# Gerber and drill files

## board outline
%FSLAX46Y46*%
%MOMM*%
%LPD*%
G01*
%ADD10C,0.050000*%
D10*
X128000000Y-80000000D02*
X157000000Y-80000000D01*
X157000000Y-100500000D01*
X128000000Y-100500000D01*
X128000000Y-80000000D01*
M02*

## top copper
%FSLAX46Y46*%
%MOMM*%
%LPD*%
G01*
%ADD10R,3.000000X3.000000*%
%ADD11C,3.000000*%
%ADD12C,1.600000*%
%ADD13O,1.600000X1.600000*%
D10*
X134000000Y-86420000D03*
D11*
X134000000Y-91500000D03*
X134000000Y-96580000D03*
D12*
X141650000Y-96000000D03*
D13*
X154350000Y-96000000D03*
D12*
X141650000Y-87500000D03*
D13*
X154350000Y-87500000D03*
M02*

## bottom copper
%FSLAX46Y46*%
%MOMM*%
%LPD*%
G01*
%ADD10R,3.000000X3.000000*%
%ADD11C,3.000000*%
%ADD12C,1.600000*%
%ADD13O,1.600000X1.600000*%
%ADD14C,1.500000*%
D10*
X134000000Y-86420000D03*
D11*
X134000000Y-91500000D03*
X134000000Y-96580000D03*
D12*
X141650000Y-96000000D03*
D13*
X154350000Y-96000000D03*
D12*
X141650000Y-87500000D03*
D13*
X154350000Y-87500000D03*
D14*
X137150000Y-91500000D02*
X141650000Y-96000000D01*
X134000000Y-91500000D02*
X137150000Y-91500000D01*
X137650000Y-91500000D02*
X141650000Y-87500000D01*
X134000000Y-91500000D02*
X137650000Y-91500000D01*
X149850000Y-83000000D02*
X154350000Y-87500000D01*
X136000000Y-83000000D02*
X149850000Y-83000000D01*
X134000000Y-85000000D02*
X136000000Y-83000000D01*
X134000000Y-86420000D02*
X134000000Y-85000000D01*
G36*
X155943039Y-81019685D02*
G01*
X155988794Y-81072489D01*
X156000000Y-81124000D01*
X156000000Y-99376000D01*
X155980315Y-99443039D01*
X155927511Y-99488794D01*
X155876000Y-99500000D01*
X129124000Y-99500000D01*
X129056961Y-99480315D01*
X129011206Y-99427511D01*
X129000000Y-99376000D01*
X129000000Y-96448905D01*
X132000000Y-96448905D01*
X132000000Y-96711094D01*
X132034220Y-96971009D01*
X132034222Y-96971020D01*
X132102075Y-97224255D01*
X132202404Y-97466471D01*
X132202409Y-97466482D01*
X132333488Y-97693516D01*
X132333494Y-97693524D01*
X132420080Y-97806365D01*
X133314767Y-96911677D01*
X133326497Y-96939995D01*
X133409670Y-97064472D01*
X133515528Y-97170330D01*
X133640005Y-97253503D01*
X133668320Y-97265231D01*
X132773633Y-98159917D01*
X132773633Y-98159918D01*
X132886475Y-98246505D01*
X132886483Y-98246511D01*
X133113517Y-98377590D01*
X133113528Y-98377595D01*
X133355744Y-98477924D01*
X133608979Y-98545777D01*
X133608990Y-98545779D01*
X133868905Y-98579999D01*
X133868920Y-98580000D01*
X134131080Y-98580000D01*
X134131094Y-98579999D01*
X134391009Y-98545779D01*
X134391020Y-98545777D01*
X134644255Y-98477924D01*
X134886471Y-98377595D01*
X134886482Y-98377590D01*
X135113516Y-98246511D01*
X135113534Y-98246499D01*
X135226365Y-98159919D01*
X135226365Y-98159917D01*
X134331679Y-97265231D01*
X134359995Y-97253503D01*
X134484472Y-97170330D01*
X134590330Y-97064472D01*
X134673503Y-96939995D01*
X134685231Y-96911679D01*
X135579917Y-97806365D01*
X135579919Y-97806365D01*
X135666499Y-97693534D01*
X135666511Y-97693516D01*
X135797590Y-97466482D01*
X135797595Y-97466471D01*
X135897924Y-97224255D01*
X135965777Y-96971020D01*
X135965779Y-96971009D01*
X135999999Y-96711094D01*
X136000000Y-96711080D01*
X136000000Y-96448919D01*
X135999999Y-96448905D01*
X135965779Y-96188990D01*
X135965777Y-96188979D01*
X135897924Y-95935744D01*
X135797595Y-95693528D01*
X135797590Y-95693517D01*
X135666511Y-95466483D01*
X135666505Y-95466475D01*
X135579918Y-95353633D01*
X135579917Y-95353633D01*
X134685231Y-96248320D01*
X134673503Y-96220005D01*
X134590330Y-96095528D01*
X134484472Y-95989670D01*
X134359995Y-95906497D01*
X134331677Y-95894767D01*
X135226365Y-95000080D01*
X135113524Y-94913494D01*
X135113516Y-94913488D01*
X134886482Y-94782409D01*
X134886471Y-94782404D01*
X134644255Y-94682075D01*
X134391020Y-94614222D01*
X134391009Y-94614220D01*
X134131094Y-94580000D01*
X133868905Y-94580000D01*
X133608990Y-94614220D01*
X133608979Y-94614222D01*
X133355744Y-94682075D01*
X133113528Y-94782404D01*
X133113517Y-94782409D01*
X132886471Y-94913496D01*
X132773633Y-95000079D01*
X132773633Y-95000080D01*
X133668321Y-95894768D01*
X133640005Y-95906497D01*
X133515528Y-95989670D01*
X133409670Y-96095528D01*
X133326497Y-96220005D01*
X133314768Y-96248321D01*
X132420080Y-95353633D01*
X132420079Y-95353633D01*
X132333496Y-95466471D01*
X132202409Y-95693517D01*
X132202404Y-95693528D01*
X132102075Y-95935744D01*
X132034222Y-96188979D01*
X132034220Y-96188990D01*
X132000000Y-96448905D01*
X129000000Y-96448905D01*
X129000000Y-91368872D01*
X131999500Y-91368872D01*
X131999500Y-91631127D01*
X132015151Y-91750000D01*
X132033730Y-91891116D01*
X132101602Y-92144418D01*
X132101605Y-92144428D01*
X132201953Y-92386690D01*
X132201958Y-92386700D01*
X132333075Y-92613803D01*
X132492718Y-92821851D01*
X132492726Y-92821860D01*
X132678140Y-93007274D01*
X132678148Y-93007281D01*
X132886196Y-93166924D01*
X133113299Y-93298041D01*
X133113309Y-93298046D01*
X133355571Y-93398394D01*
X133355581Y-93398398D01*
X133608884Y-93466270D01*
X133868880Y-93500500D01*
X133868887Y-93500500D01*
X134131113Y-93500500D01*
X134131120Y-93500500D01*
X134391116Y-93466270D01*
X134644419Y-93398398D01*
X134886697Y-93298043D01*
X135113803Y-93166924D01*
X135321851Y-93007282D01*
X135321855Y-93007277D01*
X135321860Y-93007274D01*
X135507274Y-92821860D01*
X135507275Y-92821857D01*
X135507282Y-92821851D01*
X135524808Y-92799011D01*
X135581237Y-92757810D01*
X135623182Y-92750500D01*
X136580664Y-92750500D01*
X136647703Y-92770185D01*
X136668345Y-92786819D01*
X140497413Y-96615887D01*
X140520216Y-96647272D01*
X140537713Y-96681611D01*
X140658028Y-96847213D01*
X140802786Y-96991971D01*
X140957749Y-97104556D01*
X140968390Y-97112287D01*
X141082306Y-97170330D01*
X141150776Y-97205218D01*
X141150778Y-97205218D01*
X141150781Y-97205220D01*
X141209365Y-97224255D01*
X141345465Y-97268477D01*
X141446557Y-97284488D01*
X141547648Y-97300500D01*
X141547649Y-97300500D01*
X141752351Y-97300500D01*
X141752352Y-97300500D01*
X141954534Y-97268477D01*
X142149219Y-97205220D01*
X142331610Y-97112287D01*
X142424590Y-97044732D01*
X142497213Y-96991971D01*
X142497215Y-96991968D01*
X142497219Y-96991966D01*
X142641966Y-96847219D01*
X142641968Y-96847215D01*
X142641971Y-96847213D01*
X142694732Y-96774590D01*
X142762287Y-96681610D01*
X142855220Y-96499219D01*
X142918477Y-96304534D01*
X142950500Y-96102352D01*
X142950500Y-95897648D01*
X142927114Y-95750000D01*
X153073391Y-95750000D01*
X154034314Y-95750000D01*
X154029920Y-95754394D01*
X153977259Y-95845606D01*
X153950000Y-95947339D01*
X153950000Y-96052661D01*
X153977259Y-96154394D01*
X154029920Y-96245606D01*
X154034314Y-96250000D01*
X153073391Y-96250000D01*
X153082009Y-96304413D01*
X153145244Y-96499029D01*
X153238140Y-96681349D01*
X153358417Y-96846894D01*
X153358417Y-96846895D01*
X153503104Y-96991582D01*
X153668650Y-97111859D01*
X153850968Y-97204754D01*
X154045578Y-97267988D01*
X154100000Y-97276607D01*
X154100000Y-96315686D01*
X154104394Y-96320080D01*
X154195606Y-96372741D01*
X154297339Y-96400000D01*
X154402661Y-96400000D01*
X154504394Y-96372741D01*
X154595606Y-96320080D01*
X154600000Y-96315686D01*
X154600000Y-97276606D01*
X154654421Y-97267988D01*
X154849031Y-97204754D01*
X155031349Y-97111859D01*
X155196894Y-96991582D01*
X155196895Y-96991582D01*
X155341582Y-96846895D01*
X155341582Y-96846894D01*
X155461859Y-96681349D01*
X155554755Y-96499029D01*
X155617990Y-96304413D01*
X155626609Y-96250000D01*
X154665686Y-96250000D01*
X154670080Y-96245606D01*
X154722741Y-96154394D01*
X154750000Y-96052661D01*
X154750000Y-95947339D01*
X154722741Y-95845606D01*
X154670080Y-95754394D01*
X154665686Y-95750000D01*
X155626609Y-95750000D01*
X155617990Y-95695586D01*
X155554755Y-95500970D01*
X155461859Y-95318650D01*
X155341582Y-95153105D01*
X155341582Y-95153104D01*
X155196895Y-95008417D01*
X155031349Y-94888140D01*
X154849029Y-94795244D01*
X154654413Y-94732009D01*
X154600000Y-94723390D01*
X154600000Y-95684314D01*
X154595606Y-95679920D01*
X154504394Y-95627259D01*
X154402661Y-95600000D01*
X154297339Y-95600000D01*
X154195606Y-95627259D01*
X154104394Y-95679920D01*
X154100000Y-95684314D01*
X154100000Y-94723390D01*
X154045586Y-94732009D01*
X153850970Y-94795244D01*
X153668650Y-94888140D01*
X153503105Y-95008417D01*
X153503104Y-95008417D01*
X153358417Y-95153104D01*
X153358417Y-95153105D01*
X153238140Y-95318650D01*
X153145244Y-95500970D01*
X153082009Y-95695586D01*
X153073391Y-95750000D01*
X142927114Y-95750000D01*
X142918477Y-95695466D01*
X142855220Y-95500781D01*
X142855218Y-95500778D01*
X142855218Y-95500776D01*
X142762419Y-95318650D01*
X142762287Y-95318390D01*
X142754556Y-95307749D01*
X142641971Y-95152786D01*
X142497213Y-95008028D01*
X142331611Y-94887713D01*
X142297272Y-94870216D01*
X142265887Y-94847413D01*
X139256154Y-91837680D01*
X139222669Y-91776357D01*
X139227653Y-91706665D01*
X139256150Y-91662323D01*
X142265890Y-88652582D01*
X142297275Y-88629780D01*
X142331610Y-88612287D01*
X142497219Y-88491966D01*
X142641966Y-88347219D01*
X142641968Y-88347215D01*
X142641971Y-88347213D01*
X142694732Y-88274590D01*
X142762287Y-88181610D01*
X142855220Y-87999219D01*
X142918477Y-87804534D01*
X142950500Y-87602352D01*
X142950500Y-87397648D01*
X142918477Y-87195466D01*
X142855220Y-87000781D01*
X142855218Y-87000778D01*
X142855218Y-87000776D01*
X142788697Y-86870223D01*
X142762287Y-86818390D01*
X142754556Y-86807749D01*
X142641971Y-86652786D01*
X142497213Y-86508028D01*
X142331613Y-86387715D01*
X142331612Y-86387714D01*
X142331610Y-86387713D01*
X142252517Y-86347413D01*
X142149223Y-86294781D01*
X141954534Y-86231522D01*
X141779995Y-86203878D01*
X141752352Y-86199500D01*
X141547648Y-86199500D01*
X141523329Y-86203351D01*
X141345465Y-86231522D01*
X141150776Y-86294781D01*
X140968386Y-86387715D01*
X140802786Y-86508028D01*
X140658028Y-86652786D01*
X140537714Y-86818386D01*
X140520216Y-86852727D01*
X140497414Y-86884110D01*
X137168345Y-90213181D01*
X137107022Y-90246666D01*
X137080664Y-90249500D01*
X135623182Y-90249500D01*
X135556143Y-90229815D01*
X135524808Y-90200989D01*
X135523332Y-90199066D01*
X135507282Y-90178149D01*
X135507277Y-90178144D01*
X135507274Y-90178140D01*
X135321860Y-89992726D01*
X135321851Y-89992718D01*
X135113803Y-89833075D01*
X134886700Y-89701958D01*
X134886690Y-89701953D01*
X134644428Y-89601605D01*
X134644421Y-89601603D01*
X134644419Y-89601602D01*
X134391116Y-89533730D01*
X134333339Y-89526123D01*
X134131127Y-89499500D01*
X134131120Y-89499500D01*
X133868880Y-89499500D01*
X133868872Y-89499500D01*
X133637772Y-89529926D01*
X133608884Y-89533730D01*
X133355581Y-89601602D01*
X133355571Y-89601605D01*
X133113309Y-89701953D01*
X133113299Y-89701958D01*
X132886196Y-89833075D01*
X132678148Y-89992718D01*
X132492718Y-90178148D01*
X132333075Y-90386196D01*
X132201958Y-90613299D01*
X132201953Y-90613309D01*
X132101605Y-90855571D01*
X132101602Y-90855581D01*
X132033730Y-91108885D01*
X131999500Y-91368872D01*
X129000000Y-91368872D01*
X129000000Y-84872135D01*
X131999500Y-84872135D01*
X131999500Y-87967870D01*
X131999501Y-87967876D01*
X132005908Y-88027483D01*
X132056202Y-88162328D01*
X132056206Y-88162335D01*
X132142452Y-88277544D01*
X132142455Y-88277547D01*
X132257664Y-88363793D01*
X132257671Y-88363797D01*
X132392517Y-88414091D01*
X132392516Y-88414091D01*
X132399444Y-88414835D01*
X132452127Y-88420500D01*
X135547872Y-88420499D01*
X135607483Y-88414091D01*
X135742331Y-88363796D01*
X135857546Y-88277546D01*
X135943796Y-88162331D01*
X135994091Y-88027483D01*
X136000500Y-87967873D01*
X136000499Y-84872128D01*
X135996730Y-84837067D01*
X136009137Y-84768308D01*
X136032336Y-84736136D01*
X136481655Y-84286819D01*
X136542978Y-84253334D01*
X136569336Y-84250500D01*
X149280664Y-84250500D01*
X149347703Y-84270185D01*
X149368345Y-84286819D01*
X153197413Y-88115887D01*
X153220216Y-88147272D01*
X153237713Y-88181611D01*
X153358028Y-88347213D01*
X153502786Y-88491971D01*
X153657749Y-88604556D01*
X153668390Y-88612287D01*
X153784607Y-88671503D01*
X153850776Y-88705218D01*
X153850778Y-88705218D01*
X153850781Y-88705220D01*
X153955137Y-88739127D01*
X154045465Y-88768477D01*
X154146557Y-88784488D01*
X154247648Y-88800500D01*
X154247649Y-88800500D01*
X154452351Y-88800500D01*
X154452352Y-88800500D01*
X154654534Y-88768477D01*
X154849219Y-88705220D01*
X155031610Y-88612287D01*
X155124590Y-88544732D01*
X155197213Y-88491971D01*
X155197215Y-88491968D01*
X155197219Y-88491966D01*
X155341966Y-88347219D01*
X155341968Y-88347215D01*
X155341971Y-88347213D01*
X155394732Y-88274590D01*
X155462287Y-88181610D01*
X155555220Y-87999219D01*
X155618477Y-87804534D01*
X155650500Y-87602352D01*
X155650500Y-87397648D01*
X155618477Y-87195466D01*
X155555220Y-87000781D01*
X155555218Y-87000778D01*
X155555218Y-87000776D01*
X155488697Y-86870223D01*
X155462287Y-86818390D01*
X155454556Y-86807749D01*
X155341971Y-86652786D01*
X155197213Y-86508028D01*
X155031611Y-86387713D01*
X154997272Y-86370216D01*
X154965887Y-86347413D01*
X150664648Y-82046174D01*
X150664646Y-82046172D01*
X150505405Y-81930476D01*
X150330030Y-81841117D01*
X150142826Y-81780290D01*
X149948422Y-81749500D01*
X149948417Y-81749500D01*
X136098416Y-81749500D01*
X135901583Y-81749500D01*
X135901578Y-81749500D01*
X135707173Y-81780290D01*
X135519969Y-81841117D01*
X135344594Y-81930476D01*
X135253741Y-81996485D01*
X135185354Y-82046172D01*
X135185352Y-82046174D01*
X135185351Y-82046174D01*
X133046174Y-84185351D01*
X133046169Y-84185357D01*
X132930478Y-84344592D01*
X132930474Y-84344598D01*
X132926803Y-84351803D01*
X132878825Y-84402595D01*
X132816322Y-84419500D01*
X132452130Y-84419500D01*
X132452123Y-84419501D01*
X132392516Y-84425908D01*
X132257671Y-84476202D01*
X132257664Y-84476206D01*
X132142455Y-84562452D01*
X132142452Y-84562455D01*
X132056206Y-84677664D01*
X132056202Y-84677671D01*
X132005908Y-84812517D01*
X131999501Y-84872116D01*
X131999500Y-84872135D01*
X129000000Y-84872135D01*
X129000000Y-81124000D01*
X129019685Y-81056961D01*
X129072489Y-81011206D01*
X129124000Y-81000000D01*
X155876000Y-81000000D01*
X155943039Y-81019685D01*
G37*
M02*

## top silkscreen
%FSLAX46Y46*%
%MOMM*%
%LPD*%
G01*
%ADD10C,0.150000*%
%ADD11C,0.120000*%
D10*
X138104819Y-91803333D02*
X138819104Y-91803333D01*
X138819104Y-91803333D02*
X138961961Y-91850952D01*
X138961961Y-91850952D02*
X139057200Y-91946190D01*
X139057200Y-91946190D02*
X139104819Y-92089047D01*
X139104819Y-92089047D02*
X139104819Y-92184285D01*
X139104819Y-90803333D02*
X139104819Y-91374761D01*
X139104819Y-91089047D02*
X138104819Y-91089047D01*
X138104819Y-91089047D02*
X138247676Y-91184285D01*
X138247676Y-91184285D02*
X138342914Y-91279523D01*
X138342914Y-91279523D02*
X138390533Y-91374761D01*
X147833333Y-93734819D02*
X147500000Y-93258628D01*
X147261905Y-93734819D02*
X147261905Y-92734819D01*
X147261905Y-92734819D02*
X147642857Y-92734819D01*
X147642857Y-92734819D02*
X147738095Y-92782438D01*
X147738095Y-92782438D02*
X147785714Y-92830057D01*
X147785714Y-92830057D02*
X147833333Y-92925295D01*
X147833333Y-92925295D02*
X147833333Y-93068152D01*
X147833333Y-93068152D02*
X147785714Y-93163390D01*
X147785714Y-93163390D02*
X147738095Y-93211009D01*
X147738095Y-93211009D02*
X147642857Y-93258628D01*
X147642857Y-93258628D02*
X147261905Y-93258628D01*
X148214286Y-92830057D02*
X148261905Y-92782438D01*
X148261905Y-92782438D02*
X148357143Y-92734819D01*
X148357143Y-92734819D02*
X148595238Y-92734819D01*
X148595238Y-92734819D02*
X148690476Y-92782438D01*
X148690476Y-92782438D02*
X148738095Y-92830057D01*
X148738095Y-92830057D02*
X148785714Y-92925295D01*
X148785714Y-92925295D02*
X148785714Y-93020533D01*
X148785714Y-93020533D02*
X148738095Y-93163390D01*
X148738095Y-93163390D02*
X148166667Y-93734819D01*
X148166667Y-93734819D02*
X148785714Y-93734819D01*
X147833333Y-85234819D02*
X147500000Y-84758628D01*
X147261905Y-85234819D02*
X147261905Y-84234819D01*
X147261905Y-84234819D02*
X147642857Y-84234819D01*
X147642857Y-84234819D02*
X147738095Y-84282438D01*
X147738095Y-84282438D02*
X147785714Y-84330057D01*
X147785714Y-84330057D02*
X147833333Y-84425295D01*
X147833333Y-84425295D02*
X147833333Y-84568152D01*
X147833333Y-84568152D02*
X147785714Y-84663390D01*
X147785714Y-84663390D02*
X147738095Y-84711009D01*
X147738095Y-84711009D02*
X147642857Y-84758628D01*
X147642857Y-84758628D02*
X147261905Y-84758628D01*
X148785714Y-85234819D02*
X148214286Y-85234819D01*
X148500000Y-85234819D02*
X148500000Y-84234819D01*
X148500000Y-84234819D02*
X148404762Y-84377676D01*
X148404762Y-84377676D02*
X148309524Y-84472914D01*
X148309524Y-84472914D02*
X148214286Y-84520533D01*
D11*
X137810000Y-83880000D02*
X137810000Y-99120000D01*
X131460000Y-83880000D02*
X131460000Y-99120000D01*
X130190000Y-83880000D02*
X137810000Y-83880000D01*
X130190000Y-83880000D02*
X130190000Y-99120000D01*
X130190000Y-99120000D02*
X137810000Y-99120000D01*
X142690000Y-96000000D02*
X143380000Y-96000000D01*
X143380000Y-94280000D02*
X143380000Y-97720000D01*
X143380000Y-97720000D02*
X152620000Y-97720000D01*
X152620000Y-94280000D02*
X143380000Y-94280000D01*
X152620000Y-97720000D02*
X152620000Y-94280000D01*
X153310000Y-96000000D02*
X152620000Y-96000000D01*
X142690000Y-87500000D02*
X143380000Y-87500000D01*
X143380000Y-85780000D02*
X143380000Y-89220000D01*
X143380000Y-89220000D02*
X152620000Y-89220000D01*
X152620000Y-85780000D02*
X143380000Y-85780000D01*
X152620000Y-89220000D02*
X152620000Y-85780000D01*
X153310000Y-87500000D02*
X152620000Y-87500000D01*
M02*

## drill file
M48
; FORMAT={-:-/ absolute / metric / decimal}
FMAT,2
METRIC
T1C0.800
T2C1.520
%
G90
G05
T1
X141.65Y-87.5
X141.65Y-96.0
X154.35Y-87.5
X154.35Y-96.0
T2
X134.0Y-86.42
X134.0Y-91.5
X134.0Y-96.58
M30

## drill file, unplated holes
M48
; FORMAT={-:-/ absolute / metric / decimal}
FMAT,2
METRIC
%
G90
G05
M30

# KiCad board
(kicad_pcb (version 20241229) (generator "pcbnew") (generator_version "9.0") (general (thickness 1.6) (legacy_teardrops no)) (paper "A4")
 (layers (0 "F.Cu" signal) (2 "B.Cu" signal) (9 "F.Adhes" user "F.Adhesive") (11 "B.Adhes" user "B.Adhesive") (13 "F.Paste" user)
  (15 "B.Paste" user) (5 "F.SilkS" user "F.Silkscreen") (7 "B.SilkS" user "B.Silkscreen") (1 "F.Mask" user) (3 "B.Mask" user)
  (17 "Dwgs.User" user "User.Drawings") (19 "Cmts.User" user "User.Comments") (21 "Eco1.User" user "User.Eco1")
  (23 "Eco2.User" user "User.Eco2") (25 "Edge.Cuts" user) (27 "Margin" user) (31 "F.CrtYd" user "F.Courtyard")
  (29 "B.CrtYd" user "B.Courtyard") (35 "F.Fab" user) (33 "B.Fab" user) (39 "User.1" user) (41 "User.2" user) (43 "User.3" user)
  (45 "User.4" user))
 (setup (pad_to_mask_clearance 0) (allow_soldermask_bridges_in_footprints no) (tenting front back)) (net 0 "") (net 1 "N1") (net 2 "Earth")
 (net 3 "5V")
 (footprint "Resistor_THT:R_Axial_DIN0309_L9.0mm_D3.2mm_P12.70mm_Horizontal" (layer "F.Cu") (at 141.65 96)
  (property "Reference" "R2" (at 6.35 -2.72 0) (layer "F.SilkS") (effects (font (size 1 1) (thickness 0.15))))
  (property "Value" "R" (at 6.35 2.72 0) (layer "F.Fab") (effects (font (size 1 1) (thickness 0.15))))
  (fp_line (start 1.04 0) (end 1.73 0) (stroke (width 0.12) (type solid)) (layer "F.SilkS"))
  (fp_line (start 1.73 -1.72) (end 1.73 1.72) (stroke (width 0.12) (type solid)) (layer "F.SilkS"))
  (fp_line (start 1.73 1.72) (end 10.97 1.72) (stroke (width 0.12) (type solid)) (layer "F.SilkS"))
  (fp_line (start 10.97 -1.72) (end 1.73 -1.72) (stroke (width 0.12) (type solid)) (layer "F.SilkS"))
  (fp_line (start 10.97 1.72) (end 10.97 -1.72) (stroke (width 0.12) (type solid)) (layer "F.SilkS"))
  (fp_line (start 11.66 0) (end 10.97 0) (stroke (width 0.12) (type solid)) (layer "F.SilkS"))
  (pad "1" thru_hole circle (at 0 0) (size 1.6 1.6) (drill 0.8) (layers "*.Cu" "*.Mask") (remove_unused_layers no) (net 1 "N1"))
  (pad "2" thru_hole oval (at 12.7 0) (size 1.6 1.6) (drill 0.8) (layers "*.Cu" "*.Mask") (remove_unused_layers no) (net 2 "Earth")))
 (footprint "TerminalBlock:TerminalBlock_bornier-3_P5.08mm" (layer "F.Cu") (at 134 86.42 -90)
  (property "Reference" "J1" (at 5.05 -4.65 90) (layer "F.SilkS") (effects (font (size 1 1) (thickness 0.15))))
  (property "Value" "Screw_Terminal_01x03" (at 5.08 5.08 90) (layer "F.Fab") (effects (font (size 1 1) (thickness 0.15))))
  (fp_line (start -2.54 3.81) (end 12.7 3.81) (stroke (width 0.12) (type solid)) (layer "F.SilkS"))
  (fp_line (start -2.54 3.81) (end -2.54 -3.81) (stroke (width 0.12) (type solid)) (layer "F.SilkS"))
  (fp_line (start 12.7 3.81) (end 12.7 -3.81) (stroke (width 0.12) (type solid)) (layer "F.SilkS"))
  (fp_line (start -2.54 2.54) (end 12.7 2.54) (stroke (width 0.12) (type solid)) (layer "F.SilkS"))
  (fp_line (start -2.54 -3.81) (end 12.7 -3.81) (stroke (width 0.12) (type solid)) (layer "F.SilkS"))
  (pad "1" thru_hole rect (at 0 0 270) (size 3 3) (drill 1.52) (layers "*.Cu" "*.Mask") (remove_unused_layers no) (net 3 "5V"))
  (pad "2" thru_hole circle (at 5.08 0 270) (size 3 3) (drill 1.52) (layers "*.Cu" "*.Mask") (remove_unused_layers no) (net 1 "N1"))
  (pad "3" thru_hole circle (at 10.16 0 270) (size 3 3) (drill 1.52) (layers "*.Cu" "*.Mask") (remove_unused_layers no) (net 2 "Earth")))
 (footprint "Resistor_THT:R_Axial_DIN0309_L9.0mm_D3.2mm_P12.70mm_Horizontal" (layer "F.Cu") (at 141.65 87.5)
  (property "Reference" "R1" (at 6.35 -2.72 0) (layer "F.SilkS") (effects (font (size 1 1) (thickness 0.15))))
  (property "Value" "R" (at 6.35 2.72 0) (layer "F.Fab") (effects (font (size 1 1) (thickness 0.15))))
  (fp_line (start 1.04 0) (end 1.73 0) (stroke (width 0.12) (type solid)) (layer "F.SilkS"))
  (fp_line (start 1.73 -1.72) (end 1.73 1.72) (stroke (width 0.12) (type solid)) (layer "F.SilkS"))
  (fp_line (start 1.73 1.72) (end 10.97 1.72) (stroke (width 0.12) (type solid)) (layer "F.SilkS"))
  (fp_line (start 10.97 -1.72) (end 1.73 -1.72) (stroke (width 0.12) (type solid)) (layer "F.SilkS"))
  (fp_line (start 10.97 1.72) (end 10.97 -1.72) (stroke (width 0.12) (type solid)) (layer "F.SilkS"))
  (fp_line (start 11.66 0) (end 10.97 0) (stroke (width 0.12) (type solid)) (layer "F.SilkS"))
  (pad "1" thru_hole circle (at 0 0) (size 1.6 1.6) (drill 0.8) (layers "*.Cu" "*.Mask") (remove_unused_layers no) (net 1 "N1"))
  (pad "2" thru_hole oval (at 12.7 0) (size 1.6 1.6) (drill 0.8) (layers "*.Cu" "*.Mask") (remove_unused_layers no) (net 3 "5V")))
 (gr_rect (start 128 80) (end 157 100.5) (stroke (width 0.05) (type default)) (fill no) (layer "Edge.Cuts"))
 (segment (start 134 85) (end 136 83) (width 1.5) (layer "B.Cu") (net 3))
 (segment (start 134 86.42) (end 134 85) (width 1.5) (layer "B.Cu") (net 3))
 (segment (start 136 83) (end 149.85 83) (width 1.5) (layer "B.Cu") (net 3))
 (segment (start 149.85 83) (end 154.35 87.5) (width 1.5) (layer "B.Cu") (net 3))
 (segment (start 137.15 91.5) (end 141.65 96) (width 1.5) (layer "B.Cu") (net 1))
 (segment (start 137.65 91.5) (end 141.65 87.5) (width 1.5) (layer "B.Cu") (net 1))
 (segment (start 134 91.5) (end 137.15 91.5) (width 1.5) (layer "B.Cu") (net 1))
 (segment (start 134 91.5) (end 137.65 91.5) (width 1.5) (layer "B.Cu") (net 1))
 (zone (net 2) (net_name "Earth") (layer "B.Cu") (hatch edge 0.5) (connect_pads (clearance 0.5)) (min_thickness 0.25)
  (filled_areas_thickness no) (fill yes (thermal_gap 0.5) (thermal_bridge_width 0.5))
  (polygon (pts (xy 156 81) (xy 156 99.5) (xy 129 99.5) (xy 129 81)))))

